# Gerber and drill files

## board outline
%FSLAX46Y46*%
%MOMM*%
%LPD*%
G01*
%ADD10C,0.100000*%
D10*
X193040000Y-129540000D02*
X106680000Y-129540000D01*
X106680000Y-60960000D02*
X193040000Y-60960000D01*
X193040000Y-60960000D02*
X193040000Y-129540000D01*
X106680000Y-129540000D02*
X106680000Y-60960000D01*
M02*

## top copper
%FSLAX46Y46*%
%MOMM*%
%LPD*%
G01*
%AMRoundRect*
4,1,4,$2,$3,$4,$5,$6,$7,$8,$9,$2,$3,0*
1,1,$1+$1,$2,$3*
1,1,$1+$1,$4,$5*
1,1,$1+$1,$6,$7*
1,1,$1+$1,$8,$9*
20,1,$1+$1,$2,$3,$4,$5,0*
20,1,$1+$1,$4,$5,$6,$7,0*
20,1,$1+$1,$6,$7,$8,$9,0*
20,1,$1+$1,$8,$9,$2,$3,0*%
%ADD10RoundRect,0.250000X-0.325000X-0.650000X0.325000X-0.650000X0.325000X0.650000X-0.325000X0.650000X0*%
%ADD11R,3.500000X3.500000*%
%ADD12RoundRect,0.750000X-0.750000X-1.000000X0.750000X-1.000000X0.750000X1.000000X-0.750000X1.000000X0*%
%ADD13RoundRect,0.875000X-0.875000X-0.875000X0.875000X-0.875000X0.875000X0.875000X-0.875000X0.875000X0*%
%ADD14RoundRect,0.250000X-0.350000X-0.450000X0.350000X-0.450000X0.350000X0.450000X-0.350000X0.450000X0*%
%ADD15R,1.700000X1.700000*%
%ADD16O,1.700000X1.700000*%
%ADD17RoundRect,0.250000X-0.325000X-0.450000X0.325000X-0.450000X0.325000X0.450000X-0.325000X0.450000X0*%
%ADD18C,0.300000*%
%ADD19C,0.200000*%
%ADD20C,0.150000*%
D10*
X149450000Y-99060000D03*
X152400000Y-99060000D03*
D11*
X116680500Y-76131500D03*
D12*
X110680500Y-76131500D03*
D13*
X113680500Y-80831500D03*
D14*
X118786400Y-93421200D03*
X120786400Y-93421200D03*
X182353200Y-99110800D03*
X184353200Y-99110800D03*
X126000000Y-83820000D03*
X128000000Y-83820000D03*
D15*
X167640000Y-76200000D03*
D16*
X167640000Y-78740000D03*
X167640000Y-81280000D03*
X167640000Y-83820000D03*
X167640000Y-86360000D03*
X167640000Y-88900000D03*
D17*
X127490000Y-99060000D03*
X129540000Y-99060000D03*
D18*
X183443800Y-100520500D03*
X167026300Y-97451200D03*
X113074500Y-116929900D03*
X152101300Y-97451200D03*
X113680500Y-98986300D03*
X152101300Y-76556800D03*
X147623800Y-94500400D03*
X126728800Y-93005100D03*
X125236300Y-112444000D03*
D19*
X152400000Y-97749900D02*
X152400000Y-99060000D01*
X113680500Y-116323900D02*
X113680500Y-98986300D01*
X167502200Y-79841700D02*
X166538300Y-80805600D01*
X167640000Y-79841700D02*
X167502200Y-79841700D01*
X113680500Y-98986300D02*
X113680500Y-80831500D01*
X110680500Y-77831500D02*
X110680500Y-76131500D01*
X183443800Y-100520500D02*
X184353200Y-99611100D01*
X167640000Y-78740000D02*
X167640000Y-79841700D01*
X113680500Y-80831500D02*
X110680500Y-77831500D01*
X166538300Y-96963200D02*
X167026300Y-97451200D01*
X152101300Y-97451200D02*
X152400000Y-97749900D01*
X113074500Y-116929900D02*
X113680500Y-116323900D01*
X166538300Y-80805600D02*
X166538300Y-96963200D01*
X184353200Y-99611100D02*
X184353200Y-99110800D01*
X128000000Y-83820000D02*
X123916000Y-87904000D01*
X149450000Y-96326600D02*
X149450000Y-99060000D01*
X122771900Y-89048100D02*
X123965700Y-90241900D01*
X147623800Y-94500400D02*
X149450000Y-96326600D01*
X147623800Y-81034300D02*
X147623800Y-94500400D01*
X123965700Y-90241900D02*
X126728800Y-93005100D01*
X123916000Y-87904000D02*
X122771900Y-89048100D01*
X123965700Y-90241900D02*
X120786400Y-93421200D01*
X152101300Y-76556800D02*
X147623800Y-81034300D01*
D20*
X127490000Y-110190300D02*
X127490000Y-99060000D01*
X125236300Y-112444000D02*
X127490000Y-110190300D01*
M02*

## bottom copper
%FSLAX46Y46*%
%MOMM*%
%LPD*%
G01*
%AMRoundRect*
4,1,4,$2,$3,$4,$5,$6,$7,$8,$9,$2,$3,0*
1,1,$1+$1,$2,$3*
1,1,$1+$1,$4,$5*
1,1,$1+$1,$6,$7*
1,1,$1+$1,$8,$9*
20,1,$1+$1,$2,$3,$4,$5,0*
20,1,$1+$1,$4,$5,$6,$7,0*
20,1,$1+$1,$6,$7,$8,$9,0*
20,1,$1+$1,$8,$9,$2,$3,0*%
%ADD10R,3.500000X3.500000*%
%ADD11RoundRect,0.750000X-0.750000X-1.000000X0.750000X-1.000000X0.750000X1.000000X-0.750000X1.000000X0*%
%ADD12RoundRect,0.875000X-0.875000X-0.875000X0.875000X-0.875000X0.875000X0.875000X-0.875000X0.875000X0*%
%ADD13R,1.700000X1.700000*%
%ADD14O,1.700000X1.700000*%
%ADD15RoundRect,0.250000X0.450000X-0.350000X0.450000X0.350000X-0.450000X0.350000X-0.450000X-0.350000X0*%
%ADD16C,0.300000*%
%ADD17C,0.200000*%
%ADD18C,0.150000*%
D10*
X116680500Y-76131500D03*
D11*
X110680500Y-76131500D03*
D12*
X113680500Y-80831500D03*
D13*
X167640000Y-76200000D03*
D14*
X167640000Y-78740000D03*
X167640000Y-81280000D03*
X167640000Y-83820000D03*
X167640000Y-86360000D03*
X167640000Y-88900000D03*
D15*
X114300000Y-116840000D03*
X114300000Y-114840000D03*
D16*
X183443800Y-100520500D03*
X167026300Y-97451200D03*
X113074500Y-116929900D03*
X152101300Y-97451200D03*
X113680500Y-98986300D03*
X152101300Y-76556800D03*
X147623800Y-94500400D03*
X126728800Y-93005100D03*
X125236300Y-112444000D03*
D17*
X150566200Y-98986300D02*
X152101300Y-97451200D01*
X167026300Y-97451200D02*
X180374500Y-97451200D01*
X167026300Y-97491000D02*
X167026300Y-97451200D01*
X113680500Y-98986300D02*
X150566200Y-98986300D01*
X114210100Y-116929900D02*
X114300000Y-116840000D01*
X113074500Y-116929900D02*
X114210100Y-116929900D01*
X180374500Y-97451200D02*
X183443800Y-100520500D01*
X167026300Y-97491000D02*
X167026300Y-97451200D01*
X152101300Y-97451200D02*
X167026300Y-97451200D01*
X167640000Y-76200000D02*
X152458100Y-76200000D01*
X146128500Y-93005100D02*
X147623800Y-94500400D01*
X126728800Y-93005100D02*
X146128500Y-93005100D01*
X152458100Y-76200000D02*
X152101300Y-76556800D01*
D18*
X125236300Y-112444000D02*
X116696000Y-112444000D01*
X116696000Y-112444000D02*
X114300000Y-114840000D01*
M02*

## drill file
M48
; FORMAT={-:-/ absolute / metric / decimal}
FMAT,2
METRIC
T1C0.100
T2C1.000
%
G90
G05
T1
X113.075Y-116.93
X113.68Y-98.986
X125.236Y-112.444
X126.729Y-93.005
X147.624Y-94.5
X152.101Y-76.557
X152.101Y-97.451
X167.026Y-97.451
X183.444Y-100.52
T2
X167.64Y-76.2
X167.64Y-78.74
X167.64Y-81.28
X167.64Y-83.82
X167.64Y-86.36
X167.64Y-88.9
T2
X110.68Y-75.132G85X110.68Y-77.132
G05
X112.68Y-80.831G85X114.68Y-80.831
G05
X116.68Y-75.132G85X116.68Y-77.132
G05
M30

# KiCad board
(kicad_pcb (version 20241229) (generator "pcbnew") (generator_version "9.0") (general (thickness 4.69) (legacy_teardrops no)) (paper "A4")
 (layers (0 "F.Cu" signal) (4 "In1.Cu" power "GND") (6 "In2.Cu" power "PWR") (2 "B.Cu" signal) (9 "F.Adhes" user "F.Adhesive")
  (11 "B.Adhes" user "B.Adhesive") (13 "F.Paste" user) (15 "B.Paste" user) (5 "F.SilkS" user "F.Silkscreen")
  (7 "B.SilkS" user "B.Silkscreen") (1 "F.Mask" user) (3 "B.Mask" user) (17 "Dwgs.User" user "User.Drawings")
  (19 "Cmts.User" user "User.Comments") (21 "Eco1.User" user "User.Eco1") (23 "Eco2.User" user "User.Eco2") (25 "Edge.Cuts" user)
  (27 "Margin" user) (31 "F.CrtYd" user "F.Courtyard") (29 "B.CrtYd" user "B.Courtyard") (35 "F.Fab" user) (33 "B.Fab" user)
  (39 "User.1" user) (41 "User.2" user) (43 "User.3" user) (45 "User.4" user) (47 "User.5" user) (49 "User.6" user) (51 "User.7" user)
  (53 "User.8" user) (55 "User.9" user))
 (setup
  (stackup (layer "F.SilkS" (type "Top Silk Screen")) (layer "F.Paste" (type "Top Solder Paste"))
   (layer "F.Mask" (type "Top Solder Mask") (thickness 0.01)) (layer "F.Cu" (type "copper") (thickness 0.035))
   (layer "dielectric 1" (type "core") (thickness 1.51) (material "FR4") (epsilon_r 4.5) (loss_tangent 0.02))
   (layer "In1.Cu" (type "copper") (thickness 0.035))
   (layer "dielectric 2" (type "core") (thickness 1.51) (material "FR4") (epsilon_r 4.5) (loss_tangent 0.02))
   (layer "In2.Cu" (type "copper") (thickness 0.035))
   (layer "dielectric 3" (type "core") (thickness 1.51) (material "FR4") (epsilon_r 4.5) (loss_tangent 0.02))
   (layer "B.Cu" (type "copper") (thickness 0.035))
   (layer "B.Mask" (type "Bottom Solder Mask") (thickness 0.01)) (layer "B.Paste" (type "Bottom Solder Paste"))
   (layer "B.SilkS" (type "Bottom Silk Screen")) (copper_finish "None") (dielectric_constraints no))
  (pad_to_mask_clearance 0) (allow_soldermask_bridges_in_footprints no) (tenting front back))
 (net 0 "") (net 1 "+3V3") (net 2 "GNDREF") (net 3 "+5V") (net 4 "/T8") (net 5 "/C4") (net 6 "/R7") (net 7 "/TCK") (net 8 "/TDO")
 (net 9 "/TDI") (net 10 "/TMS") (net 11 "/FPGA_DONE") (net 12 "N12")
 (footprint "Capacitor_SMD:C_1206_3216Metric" (layer "F.Cu") (at 150.925 99.06)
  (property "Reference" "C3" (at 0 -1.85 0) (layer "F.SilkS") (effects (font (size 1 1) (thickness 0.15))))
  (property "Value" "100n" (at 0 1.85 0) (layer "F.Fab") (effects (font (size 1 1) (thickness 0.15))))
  (pad "1" smd roundrect (at -1.475 0) (size 1.15 1.8) (layers "F.Cu" "F.Mask" "F.Paste") (roundrect_rratio 0.217391) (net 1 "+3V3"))
  (pad "2" smd roundrect (at 1.475 0) (size 1.15 1.8) (layers "F.Cu" "F.Mask" "F.Paste") (roundrect_rratio 0.217391) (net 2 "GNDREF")))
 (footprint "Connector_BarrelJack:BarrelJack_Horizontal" (layer "F.Cu") (at 116.6805 76.1315)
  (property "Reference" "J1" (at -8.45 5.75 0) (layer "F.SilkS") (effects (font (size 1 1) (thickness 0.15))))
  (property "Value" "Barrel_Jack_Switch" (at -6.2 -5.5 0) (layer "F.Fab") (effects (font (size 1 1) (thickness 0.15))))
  (pad "1" thru_hole rect (at 0 0) (size 3.5 3.5) (drill oval 1 3) (layers "*.Cu" "*.Mask") (remove_unused_layers no) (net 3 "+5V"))
  (pad "2" thru_hole roundrect (at -6 0) (size 3 3.5) (drill oval 1 3) (layers "*.Cu" "*.Mask") (remove_unused_layers no)
   (roundrect_rratio 0.25) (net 2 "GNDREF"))
  (pad "3" thru_hole roundrect (at -3 4.7) (size 3.5 3.5) (drill oval 3 1) (layers "*.Cu" "*.Mask") (remove_unused_layers no)
   (roundrect_rratio 0.25) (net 2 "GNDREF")))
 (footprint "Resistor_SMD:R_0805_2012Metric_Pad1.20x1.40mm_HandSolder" (layer "F.Cu") (at 119.7864 93.4212)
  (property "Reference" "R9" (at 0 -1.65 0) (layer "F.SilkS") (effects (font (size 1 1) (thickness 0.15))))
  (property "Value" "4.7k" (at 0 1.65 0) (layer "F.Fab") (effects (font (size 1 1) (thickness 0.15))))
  (pad "1" smd roundrect (at -1 0) (size 1.2 1.4) (layers "F.Cu" "F.Mask" "F.Paste") (roundrect_rratio 0.208333) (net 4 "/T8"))
  (pad "2" smd roundrect (at 1 0) (size 1.2 1.4) (layers "F.Cu" "F.Mask" "F.Paste") (roundrect_rratio 0.208333) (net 1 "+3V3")))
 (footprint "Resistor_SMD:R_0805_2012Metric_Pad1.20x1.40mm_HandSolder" (layer "F.Cu") (at 183.3532 99.1108)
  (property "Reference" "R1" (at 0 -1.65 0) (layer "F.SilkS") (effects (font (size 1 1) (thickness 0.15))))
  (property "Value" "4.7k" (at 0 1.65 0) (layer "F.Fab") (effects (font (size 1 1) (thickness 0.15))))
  (pad "1" smd roundrect (at -1 0) (size 1.2 1.4) (layers "F.Cu" "F.Mask" "F.Paste") (roundrect_rratio 0.208333) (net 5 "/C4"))
  (pad "2" smd roundrect (at 1 0) (size 1.2 1.4) (layers "F.Cu" "F.Mask" "F.Paste") (roundrect_rratio 0.208333) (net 2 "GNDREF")))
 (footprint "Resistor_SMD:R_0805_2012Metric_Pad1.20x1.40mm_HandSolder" (layer "F.Cu") (at 127 83.82)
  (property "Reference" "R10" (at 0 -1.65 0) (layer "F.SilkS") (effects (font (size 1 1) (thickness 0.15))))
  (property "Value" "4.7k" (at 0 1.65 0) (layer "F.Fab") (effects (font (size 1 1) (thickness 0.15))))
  (pad "1" smd roundrect (at -1 0) (size 1.2 1.4) (layers "F.Cu" "F.Mask" "F.Paste") (roundrect_rratio 0.208333) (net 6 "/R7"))
  (pad "2" smd roundrect (at 1 0) (size 1.2 1.4) (layers "F.Cu" "F.Mask" "F.Paste") (roundrect_rratio 0.208333) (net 1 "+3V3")))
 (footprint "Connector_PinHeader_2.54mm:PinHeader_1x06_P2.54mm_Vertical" (layer "F.Cu") (at 167.64 76.2)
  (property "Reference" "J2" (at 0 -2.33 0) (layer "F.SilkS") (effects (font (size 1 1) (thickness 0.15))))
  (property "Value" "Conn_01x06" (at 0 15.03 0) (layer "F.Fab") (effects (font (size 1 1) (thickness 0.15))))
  (pad "1" thru_hole rect (at 0 0) (size 1.7 1.7) (drill 1) (layers "*.Cu" "*.Mask") (remove_unused_layers no) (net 1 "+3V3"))
  (pad "2" thru_hole oval (at 0 2.54) (size 1.7 1.7) (drill 1) (layers "*.Cu" "*.Mask") (remove_unused_layers no) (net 2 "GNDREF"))
  (pad "3" thru_hole oval (at 0 5.08) (size 1.7 1.7) (drill 1) (layers "*.Cu" "*.Mask") (remove_unused_layers no) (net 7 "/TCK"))
  (pad "4" thru_hole oval (at 0 7.62) (size 1.7 1.7) (drill 1) (layers "*.Cu" "*.Mask") (remove_unused_layers no) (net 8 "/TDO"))
  (pad "5" thru_hole oval (at 0 10.16) (size 1.7 1.7) (drill 1) (layers "*.Cu" "*.Mask") (remove_unused_layers no) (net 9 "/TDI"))
  (pad "6" thru_hole oval (at 0 12.7) (size 1.7 1.7) (drill 1) (layers "*.Cu" "*.Mask") (remove_unused_layers no) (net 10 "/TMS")))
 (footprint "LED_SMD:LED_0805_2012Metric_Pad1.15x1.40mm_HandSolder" (layer "F.Cu") (at 128.515 99.06)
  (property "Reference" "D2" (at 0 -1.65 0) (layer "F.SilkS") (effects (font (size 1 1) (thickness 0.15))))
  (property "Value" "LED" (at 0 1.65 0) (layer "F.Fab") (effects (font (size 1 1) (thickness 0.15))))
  (pad "1" smd roundrect (at -1.025 0) (size 1.15 1.4) (layers "F.Cu" "F.Mask" "F.Paste") (roundrect_rratio 0.217391) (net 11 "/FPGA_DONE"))
  (pad "2" smd roundrect (at 1.025 0) (size 1.15 1.4) (layers "F.Cu" "F.Mask" "F.Paste") (roundrect_rratio 0.217391) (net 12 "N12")))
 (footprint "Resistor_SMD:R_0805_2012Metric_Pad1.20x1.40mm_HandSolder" (layer "B.Cu") (at 114.3 115.84 90)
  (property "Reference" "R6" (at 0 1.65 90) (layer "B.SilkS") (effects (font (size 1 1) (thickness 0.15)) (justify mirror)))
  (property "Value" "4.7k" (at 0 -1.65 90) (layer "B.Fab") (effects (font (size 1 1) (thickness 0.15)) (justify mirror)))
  (pad "1" smd roundrect (at -1 0 90) (size 1.2 1.4) (layers "B.Cu" "B.Mask" "B.Paste") (roundrect_rratio 0.208333) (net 2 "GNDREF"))
  (pad "2" smd roundrect (at 1 0 90) (size 1.2 1.4) (layers "B.Cu" "B.Mask" "B.Paste") (roundrect_rratio 0.208333) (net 11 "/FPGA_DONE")))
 (gr_line (start 193.04 129.54) (end 106.68 129.54) (stroke (width 0.1) (type solid)) (layer "Edge.Cuts"))
 (gr_line (start 106.68 60.96) (end 193.04 60.96) (stroke (width 0.1) (type solid)) (layer "Edge.Cuts"))
 (gr_line (start 193.04 60.96) (end 193.04 129.54) (stroke (width 0.1) (type solid)) (layer "Edge.Cuts"))
 (gr_line (start 106.68 129.54) (end 106.68 60.96) (stroke (width 0.1) (type solid)) (layer "Edge.Cuts"))
 (segment (start 152.4 97.7499) (end 152.4 99.06) (width 0.2) (layer "F.Cu") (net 2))
 (segment (start 113.6805 116.3239) (end 113.6805 98.9863) (width 0.2) (layer "F.Cu") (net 2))
 (segment (start 167.5022 79.8417) (end 166.5383 80.8056) (width 0.2) (layer "F.Cu") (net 2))
 (segment (start 167.64 79.8417) (end 167.5022 79.8417) (width 0.2) (layer "F.Cu") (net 2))
 (segment (start 113.6805 98.9863) (end 113.6805 80.8315) (width 0.2) (layer "F.Cu") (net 2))
 (segment (start 110.6805 77.8315) (end 110.6805 76.1315) (width 0.2) (layer "F.Cu") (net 2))
 (segment (start 183.4438 100.5205) (end 184.3532 99.6111) (width 0.2) (layer "F.Cu") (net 2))
 (segment (start 167.64 78.74) (end 167.64 79.8417) (width 0.2) (layer "F.Cu") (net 2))
 (segment (start 113.6805 80.8315) (end 110.6805 77.8315) (width 0.2) (layer "F.Cu") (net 2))
 (segment (start 166.5383 96.9632) (end 167.0263 97.4512) (width 0.2) (layer "F.Cu") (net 2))
 (segment (start 152.1013 97.4512) (end 152.4 97.7499) (width 0.2) (layer "F.Cu") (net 2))
 (segment (start 113.0745 116.9299) (end 113.6805 116.3239) (width 0.2) (layer "F.Cu") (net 2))
 (segment (start 166.5383 80.8056) (end 166.5383 96.9632) (width 0.2) (layer "F.Cu") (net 2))
 (segment (start 184.3532 99.6111) (end 184.3532 99.1108) (width 0.2) (layer "F.Cu") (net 2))
 (via (at 183.4438 100.5205) (size 0.3) (drill 0.1) (layers "F.Cu" "B.Cu") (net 2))
 (via (at 167.0263 97.4512) (size 0.3) (drill 0.1) (layers "F.Cu" "B.Cu") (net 2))
 (via (at 113.0745 116.9299) (size 0.3) (drill 0.1) (layers "F.Cu" "B.Cu") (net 2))
 (via (at 152.1013 97.4512) (size 0.3) (drill 0.1) (layers "F.Cu" "B.Cu") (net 2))
 (via (at 113.6805 98.9863) (size 0.3) (drill 0.1) (layers "F.Cu" "B.Cu") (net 2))
 (segment (start 150.5662 98.9863) (end 152.1013 97.4512) (width 0.2) (layer "B.Cu") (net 2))
 (segment (start 167.0263 97.4512) (end 180.3745 97.4512) (width 0.2) (layer "B.Cu") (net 2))
 (segment (start 167.0263 97.491) (end 167.0263 97.4512) (width 0.2) (layer "B.Cu") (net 2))
 (segment (start 113.6805 98.9863) (end 150.5662 98.9863) (width 0.2) (layer "B.Cu") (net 2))
 (segment (start 114.2101 116.9299) (end 114.3 116.84) (width 0.2) (layer "B.Cu") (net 2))
 (segment (start 113.0745 116.9299) (end 114.2101 116.9299) (width 0.2) (layer "B.Cu") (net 2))
 (segment (start 180.3745 97.4512) (end 183.4438 100.5205) (width 0.2) (layer "B.Cu") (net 2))
 (segment (start 167.0263 97.491) (end 167.0263 97.4512) (width 0.2) (layer "B.Cu") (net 2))
 (segment (start 152.1013 97.4512) (end 167.0263 97.4512) (width 0.2) (layer "B.Cu") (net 2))
 (segment (start 128 83.82) (end 123.916 87.904) (width 0.2) (layer "F.Cu") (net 1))
 (segment (start 149.45 96.3266) (end 149.45 99.06) (width 0.2) (layer "F.Cu") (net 1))
 (segment (start 122.7719 89.0481) (end 123.9657 90.2419) (width 0.2) (layer "F.Cu") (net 1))
 (segment (start 147.6238 94.5004) (end 149.45 96.3266) (width 0.2) (layer "F.Cu") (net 1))
 (segment (start 147.6238 81.0343) (end 147.6238 94.5004) (width 0.2) (layer "F.Cu") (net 1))
 (segment (start 123.9657 90.2419) (end 126.7288 93.0051) (width 0.2) (layer "F.Cu") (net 1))
 (segment (start 123.916 87.904) (end 122.7719 89.0481) (width 0.2) (layer "F.Cu") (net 1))
 (segment (start 123.9657 90.2419) (end 120.7864 93.4212) (width 0.2) (layer "F.Cu") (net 1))
 (segment (start 152.1013 76.5568) (end 147.6238 81.0343) (width 0.2) (layer "F.Cu") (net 1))
 (via (at 152.1013 76.5568) (size 0.3) (drill 0.1) (layers "F.Cu" "B.Cu") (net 1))
 (via (at 147.6238 94.5004) (size 0.3) (drill 0.1) (layers "F.Cu" "B.Cu") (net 1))
 (via (at 126.7288 93.0051) (size 0.3) (drill 0.1) (layers "F.Cu" "B.Cu") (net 1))
 (segment (start 167.64 76.2) (end 152.4581 76.2) (width 0.2) (layer "B.Cu") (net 1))
 (segment (start 146.1285 93.0051) (end 147.6238 94.5004) (width 0.2) (layer "B.Cu") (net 1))
 (segment (start 126.7288 93.0051) (end 146.1285 93.0051) (width 0.2) (layer "B.Cu") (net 1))
 (segment (start 152.4581 76.2) (end 152.1013 76.5568) (width 0.2) (layer "B.Cu") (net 1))
 (segment (start 127.49 110.1903) (end 127.49 99.06) (width 0.15) (layer "F.Cu") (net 11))
 (segment (start 125.2363 112.444) (end 127.49 110.1903) (width 0.15) (layer "F.Cu") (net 11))
 (via (at 125.2363 112.444) (size 0.3) (drill 0.1) (layers "F.Cu" "B.Cu") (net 11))
 (segment (start 125.2363 112.444) (end 116.696 112.444) (width 0.15) (layer "B.Cu") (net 11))
 (segment (start 116.696 112.444) (end 114.3 114.84) (width 0.15) (layer "B.Cu") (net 11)))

